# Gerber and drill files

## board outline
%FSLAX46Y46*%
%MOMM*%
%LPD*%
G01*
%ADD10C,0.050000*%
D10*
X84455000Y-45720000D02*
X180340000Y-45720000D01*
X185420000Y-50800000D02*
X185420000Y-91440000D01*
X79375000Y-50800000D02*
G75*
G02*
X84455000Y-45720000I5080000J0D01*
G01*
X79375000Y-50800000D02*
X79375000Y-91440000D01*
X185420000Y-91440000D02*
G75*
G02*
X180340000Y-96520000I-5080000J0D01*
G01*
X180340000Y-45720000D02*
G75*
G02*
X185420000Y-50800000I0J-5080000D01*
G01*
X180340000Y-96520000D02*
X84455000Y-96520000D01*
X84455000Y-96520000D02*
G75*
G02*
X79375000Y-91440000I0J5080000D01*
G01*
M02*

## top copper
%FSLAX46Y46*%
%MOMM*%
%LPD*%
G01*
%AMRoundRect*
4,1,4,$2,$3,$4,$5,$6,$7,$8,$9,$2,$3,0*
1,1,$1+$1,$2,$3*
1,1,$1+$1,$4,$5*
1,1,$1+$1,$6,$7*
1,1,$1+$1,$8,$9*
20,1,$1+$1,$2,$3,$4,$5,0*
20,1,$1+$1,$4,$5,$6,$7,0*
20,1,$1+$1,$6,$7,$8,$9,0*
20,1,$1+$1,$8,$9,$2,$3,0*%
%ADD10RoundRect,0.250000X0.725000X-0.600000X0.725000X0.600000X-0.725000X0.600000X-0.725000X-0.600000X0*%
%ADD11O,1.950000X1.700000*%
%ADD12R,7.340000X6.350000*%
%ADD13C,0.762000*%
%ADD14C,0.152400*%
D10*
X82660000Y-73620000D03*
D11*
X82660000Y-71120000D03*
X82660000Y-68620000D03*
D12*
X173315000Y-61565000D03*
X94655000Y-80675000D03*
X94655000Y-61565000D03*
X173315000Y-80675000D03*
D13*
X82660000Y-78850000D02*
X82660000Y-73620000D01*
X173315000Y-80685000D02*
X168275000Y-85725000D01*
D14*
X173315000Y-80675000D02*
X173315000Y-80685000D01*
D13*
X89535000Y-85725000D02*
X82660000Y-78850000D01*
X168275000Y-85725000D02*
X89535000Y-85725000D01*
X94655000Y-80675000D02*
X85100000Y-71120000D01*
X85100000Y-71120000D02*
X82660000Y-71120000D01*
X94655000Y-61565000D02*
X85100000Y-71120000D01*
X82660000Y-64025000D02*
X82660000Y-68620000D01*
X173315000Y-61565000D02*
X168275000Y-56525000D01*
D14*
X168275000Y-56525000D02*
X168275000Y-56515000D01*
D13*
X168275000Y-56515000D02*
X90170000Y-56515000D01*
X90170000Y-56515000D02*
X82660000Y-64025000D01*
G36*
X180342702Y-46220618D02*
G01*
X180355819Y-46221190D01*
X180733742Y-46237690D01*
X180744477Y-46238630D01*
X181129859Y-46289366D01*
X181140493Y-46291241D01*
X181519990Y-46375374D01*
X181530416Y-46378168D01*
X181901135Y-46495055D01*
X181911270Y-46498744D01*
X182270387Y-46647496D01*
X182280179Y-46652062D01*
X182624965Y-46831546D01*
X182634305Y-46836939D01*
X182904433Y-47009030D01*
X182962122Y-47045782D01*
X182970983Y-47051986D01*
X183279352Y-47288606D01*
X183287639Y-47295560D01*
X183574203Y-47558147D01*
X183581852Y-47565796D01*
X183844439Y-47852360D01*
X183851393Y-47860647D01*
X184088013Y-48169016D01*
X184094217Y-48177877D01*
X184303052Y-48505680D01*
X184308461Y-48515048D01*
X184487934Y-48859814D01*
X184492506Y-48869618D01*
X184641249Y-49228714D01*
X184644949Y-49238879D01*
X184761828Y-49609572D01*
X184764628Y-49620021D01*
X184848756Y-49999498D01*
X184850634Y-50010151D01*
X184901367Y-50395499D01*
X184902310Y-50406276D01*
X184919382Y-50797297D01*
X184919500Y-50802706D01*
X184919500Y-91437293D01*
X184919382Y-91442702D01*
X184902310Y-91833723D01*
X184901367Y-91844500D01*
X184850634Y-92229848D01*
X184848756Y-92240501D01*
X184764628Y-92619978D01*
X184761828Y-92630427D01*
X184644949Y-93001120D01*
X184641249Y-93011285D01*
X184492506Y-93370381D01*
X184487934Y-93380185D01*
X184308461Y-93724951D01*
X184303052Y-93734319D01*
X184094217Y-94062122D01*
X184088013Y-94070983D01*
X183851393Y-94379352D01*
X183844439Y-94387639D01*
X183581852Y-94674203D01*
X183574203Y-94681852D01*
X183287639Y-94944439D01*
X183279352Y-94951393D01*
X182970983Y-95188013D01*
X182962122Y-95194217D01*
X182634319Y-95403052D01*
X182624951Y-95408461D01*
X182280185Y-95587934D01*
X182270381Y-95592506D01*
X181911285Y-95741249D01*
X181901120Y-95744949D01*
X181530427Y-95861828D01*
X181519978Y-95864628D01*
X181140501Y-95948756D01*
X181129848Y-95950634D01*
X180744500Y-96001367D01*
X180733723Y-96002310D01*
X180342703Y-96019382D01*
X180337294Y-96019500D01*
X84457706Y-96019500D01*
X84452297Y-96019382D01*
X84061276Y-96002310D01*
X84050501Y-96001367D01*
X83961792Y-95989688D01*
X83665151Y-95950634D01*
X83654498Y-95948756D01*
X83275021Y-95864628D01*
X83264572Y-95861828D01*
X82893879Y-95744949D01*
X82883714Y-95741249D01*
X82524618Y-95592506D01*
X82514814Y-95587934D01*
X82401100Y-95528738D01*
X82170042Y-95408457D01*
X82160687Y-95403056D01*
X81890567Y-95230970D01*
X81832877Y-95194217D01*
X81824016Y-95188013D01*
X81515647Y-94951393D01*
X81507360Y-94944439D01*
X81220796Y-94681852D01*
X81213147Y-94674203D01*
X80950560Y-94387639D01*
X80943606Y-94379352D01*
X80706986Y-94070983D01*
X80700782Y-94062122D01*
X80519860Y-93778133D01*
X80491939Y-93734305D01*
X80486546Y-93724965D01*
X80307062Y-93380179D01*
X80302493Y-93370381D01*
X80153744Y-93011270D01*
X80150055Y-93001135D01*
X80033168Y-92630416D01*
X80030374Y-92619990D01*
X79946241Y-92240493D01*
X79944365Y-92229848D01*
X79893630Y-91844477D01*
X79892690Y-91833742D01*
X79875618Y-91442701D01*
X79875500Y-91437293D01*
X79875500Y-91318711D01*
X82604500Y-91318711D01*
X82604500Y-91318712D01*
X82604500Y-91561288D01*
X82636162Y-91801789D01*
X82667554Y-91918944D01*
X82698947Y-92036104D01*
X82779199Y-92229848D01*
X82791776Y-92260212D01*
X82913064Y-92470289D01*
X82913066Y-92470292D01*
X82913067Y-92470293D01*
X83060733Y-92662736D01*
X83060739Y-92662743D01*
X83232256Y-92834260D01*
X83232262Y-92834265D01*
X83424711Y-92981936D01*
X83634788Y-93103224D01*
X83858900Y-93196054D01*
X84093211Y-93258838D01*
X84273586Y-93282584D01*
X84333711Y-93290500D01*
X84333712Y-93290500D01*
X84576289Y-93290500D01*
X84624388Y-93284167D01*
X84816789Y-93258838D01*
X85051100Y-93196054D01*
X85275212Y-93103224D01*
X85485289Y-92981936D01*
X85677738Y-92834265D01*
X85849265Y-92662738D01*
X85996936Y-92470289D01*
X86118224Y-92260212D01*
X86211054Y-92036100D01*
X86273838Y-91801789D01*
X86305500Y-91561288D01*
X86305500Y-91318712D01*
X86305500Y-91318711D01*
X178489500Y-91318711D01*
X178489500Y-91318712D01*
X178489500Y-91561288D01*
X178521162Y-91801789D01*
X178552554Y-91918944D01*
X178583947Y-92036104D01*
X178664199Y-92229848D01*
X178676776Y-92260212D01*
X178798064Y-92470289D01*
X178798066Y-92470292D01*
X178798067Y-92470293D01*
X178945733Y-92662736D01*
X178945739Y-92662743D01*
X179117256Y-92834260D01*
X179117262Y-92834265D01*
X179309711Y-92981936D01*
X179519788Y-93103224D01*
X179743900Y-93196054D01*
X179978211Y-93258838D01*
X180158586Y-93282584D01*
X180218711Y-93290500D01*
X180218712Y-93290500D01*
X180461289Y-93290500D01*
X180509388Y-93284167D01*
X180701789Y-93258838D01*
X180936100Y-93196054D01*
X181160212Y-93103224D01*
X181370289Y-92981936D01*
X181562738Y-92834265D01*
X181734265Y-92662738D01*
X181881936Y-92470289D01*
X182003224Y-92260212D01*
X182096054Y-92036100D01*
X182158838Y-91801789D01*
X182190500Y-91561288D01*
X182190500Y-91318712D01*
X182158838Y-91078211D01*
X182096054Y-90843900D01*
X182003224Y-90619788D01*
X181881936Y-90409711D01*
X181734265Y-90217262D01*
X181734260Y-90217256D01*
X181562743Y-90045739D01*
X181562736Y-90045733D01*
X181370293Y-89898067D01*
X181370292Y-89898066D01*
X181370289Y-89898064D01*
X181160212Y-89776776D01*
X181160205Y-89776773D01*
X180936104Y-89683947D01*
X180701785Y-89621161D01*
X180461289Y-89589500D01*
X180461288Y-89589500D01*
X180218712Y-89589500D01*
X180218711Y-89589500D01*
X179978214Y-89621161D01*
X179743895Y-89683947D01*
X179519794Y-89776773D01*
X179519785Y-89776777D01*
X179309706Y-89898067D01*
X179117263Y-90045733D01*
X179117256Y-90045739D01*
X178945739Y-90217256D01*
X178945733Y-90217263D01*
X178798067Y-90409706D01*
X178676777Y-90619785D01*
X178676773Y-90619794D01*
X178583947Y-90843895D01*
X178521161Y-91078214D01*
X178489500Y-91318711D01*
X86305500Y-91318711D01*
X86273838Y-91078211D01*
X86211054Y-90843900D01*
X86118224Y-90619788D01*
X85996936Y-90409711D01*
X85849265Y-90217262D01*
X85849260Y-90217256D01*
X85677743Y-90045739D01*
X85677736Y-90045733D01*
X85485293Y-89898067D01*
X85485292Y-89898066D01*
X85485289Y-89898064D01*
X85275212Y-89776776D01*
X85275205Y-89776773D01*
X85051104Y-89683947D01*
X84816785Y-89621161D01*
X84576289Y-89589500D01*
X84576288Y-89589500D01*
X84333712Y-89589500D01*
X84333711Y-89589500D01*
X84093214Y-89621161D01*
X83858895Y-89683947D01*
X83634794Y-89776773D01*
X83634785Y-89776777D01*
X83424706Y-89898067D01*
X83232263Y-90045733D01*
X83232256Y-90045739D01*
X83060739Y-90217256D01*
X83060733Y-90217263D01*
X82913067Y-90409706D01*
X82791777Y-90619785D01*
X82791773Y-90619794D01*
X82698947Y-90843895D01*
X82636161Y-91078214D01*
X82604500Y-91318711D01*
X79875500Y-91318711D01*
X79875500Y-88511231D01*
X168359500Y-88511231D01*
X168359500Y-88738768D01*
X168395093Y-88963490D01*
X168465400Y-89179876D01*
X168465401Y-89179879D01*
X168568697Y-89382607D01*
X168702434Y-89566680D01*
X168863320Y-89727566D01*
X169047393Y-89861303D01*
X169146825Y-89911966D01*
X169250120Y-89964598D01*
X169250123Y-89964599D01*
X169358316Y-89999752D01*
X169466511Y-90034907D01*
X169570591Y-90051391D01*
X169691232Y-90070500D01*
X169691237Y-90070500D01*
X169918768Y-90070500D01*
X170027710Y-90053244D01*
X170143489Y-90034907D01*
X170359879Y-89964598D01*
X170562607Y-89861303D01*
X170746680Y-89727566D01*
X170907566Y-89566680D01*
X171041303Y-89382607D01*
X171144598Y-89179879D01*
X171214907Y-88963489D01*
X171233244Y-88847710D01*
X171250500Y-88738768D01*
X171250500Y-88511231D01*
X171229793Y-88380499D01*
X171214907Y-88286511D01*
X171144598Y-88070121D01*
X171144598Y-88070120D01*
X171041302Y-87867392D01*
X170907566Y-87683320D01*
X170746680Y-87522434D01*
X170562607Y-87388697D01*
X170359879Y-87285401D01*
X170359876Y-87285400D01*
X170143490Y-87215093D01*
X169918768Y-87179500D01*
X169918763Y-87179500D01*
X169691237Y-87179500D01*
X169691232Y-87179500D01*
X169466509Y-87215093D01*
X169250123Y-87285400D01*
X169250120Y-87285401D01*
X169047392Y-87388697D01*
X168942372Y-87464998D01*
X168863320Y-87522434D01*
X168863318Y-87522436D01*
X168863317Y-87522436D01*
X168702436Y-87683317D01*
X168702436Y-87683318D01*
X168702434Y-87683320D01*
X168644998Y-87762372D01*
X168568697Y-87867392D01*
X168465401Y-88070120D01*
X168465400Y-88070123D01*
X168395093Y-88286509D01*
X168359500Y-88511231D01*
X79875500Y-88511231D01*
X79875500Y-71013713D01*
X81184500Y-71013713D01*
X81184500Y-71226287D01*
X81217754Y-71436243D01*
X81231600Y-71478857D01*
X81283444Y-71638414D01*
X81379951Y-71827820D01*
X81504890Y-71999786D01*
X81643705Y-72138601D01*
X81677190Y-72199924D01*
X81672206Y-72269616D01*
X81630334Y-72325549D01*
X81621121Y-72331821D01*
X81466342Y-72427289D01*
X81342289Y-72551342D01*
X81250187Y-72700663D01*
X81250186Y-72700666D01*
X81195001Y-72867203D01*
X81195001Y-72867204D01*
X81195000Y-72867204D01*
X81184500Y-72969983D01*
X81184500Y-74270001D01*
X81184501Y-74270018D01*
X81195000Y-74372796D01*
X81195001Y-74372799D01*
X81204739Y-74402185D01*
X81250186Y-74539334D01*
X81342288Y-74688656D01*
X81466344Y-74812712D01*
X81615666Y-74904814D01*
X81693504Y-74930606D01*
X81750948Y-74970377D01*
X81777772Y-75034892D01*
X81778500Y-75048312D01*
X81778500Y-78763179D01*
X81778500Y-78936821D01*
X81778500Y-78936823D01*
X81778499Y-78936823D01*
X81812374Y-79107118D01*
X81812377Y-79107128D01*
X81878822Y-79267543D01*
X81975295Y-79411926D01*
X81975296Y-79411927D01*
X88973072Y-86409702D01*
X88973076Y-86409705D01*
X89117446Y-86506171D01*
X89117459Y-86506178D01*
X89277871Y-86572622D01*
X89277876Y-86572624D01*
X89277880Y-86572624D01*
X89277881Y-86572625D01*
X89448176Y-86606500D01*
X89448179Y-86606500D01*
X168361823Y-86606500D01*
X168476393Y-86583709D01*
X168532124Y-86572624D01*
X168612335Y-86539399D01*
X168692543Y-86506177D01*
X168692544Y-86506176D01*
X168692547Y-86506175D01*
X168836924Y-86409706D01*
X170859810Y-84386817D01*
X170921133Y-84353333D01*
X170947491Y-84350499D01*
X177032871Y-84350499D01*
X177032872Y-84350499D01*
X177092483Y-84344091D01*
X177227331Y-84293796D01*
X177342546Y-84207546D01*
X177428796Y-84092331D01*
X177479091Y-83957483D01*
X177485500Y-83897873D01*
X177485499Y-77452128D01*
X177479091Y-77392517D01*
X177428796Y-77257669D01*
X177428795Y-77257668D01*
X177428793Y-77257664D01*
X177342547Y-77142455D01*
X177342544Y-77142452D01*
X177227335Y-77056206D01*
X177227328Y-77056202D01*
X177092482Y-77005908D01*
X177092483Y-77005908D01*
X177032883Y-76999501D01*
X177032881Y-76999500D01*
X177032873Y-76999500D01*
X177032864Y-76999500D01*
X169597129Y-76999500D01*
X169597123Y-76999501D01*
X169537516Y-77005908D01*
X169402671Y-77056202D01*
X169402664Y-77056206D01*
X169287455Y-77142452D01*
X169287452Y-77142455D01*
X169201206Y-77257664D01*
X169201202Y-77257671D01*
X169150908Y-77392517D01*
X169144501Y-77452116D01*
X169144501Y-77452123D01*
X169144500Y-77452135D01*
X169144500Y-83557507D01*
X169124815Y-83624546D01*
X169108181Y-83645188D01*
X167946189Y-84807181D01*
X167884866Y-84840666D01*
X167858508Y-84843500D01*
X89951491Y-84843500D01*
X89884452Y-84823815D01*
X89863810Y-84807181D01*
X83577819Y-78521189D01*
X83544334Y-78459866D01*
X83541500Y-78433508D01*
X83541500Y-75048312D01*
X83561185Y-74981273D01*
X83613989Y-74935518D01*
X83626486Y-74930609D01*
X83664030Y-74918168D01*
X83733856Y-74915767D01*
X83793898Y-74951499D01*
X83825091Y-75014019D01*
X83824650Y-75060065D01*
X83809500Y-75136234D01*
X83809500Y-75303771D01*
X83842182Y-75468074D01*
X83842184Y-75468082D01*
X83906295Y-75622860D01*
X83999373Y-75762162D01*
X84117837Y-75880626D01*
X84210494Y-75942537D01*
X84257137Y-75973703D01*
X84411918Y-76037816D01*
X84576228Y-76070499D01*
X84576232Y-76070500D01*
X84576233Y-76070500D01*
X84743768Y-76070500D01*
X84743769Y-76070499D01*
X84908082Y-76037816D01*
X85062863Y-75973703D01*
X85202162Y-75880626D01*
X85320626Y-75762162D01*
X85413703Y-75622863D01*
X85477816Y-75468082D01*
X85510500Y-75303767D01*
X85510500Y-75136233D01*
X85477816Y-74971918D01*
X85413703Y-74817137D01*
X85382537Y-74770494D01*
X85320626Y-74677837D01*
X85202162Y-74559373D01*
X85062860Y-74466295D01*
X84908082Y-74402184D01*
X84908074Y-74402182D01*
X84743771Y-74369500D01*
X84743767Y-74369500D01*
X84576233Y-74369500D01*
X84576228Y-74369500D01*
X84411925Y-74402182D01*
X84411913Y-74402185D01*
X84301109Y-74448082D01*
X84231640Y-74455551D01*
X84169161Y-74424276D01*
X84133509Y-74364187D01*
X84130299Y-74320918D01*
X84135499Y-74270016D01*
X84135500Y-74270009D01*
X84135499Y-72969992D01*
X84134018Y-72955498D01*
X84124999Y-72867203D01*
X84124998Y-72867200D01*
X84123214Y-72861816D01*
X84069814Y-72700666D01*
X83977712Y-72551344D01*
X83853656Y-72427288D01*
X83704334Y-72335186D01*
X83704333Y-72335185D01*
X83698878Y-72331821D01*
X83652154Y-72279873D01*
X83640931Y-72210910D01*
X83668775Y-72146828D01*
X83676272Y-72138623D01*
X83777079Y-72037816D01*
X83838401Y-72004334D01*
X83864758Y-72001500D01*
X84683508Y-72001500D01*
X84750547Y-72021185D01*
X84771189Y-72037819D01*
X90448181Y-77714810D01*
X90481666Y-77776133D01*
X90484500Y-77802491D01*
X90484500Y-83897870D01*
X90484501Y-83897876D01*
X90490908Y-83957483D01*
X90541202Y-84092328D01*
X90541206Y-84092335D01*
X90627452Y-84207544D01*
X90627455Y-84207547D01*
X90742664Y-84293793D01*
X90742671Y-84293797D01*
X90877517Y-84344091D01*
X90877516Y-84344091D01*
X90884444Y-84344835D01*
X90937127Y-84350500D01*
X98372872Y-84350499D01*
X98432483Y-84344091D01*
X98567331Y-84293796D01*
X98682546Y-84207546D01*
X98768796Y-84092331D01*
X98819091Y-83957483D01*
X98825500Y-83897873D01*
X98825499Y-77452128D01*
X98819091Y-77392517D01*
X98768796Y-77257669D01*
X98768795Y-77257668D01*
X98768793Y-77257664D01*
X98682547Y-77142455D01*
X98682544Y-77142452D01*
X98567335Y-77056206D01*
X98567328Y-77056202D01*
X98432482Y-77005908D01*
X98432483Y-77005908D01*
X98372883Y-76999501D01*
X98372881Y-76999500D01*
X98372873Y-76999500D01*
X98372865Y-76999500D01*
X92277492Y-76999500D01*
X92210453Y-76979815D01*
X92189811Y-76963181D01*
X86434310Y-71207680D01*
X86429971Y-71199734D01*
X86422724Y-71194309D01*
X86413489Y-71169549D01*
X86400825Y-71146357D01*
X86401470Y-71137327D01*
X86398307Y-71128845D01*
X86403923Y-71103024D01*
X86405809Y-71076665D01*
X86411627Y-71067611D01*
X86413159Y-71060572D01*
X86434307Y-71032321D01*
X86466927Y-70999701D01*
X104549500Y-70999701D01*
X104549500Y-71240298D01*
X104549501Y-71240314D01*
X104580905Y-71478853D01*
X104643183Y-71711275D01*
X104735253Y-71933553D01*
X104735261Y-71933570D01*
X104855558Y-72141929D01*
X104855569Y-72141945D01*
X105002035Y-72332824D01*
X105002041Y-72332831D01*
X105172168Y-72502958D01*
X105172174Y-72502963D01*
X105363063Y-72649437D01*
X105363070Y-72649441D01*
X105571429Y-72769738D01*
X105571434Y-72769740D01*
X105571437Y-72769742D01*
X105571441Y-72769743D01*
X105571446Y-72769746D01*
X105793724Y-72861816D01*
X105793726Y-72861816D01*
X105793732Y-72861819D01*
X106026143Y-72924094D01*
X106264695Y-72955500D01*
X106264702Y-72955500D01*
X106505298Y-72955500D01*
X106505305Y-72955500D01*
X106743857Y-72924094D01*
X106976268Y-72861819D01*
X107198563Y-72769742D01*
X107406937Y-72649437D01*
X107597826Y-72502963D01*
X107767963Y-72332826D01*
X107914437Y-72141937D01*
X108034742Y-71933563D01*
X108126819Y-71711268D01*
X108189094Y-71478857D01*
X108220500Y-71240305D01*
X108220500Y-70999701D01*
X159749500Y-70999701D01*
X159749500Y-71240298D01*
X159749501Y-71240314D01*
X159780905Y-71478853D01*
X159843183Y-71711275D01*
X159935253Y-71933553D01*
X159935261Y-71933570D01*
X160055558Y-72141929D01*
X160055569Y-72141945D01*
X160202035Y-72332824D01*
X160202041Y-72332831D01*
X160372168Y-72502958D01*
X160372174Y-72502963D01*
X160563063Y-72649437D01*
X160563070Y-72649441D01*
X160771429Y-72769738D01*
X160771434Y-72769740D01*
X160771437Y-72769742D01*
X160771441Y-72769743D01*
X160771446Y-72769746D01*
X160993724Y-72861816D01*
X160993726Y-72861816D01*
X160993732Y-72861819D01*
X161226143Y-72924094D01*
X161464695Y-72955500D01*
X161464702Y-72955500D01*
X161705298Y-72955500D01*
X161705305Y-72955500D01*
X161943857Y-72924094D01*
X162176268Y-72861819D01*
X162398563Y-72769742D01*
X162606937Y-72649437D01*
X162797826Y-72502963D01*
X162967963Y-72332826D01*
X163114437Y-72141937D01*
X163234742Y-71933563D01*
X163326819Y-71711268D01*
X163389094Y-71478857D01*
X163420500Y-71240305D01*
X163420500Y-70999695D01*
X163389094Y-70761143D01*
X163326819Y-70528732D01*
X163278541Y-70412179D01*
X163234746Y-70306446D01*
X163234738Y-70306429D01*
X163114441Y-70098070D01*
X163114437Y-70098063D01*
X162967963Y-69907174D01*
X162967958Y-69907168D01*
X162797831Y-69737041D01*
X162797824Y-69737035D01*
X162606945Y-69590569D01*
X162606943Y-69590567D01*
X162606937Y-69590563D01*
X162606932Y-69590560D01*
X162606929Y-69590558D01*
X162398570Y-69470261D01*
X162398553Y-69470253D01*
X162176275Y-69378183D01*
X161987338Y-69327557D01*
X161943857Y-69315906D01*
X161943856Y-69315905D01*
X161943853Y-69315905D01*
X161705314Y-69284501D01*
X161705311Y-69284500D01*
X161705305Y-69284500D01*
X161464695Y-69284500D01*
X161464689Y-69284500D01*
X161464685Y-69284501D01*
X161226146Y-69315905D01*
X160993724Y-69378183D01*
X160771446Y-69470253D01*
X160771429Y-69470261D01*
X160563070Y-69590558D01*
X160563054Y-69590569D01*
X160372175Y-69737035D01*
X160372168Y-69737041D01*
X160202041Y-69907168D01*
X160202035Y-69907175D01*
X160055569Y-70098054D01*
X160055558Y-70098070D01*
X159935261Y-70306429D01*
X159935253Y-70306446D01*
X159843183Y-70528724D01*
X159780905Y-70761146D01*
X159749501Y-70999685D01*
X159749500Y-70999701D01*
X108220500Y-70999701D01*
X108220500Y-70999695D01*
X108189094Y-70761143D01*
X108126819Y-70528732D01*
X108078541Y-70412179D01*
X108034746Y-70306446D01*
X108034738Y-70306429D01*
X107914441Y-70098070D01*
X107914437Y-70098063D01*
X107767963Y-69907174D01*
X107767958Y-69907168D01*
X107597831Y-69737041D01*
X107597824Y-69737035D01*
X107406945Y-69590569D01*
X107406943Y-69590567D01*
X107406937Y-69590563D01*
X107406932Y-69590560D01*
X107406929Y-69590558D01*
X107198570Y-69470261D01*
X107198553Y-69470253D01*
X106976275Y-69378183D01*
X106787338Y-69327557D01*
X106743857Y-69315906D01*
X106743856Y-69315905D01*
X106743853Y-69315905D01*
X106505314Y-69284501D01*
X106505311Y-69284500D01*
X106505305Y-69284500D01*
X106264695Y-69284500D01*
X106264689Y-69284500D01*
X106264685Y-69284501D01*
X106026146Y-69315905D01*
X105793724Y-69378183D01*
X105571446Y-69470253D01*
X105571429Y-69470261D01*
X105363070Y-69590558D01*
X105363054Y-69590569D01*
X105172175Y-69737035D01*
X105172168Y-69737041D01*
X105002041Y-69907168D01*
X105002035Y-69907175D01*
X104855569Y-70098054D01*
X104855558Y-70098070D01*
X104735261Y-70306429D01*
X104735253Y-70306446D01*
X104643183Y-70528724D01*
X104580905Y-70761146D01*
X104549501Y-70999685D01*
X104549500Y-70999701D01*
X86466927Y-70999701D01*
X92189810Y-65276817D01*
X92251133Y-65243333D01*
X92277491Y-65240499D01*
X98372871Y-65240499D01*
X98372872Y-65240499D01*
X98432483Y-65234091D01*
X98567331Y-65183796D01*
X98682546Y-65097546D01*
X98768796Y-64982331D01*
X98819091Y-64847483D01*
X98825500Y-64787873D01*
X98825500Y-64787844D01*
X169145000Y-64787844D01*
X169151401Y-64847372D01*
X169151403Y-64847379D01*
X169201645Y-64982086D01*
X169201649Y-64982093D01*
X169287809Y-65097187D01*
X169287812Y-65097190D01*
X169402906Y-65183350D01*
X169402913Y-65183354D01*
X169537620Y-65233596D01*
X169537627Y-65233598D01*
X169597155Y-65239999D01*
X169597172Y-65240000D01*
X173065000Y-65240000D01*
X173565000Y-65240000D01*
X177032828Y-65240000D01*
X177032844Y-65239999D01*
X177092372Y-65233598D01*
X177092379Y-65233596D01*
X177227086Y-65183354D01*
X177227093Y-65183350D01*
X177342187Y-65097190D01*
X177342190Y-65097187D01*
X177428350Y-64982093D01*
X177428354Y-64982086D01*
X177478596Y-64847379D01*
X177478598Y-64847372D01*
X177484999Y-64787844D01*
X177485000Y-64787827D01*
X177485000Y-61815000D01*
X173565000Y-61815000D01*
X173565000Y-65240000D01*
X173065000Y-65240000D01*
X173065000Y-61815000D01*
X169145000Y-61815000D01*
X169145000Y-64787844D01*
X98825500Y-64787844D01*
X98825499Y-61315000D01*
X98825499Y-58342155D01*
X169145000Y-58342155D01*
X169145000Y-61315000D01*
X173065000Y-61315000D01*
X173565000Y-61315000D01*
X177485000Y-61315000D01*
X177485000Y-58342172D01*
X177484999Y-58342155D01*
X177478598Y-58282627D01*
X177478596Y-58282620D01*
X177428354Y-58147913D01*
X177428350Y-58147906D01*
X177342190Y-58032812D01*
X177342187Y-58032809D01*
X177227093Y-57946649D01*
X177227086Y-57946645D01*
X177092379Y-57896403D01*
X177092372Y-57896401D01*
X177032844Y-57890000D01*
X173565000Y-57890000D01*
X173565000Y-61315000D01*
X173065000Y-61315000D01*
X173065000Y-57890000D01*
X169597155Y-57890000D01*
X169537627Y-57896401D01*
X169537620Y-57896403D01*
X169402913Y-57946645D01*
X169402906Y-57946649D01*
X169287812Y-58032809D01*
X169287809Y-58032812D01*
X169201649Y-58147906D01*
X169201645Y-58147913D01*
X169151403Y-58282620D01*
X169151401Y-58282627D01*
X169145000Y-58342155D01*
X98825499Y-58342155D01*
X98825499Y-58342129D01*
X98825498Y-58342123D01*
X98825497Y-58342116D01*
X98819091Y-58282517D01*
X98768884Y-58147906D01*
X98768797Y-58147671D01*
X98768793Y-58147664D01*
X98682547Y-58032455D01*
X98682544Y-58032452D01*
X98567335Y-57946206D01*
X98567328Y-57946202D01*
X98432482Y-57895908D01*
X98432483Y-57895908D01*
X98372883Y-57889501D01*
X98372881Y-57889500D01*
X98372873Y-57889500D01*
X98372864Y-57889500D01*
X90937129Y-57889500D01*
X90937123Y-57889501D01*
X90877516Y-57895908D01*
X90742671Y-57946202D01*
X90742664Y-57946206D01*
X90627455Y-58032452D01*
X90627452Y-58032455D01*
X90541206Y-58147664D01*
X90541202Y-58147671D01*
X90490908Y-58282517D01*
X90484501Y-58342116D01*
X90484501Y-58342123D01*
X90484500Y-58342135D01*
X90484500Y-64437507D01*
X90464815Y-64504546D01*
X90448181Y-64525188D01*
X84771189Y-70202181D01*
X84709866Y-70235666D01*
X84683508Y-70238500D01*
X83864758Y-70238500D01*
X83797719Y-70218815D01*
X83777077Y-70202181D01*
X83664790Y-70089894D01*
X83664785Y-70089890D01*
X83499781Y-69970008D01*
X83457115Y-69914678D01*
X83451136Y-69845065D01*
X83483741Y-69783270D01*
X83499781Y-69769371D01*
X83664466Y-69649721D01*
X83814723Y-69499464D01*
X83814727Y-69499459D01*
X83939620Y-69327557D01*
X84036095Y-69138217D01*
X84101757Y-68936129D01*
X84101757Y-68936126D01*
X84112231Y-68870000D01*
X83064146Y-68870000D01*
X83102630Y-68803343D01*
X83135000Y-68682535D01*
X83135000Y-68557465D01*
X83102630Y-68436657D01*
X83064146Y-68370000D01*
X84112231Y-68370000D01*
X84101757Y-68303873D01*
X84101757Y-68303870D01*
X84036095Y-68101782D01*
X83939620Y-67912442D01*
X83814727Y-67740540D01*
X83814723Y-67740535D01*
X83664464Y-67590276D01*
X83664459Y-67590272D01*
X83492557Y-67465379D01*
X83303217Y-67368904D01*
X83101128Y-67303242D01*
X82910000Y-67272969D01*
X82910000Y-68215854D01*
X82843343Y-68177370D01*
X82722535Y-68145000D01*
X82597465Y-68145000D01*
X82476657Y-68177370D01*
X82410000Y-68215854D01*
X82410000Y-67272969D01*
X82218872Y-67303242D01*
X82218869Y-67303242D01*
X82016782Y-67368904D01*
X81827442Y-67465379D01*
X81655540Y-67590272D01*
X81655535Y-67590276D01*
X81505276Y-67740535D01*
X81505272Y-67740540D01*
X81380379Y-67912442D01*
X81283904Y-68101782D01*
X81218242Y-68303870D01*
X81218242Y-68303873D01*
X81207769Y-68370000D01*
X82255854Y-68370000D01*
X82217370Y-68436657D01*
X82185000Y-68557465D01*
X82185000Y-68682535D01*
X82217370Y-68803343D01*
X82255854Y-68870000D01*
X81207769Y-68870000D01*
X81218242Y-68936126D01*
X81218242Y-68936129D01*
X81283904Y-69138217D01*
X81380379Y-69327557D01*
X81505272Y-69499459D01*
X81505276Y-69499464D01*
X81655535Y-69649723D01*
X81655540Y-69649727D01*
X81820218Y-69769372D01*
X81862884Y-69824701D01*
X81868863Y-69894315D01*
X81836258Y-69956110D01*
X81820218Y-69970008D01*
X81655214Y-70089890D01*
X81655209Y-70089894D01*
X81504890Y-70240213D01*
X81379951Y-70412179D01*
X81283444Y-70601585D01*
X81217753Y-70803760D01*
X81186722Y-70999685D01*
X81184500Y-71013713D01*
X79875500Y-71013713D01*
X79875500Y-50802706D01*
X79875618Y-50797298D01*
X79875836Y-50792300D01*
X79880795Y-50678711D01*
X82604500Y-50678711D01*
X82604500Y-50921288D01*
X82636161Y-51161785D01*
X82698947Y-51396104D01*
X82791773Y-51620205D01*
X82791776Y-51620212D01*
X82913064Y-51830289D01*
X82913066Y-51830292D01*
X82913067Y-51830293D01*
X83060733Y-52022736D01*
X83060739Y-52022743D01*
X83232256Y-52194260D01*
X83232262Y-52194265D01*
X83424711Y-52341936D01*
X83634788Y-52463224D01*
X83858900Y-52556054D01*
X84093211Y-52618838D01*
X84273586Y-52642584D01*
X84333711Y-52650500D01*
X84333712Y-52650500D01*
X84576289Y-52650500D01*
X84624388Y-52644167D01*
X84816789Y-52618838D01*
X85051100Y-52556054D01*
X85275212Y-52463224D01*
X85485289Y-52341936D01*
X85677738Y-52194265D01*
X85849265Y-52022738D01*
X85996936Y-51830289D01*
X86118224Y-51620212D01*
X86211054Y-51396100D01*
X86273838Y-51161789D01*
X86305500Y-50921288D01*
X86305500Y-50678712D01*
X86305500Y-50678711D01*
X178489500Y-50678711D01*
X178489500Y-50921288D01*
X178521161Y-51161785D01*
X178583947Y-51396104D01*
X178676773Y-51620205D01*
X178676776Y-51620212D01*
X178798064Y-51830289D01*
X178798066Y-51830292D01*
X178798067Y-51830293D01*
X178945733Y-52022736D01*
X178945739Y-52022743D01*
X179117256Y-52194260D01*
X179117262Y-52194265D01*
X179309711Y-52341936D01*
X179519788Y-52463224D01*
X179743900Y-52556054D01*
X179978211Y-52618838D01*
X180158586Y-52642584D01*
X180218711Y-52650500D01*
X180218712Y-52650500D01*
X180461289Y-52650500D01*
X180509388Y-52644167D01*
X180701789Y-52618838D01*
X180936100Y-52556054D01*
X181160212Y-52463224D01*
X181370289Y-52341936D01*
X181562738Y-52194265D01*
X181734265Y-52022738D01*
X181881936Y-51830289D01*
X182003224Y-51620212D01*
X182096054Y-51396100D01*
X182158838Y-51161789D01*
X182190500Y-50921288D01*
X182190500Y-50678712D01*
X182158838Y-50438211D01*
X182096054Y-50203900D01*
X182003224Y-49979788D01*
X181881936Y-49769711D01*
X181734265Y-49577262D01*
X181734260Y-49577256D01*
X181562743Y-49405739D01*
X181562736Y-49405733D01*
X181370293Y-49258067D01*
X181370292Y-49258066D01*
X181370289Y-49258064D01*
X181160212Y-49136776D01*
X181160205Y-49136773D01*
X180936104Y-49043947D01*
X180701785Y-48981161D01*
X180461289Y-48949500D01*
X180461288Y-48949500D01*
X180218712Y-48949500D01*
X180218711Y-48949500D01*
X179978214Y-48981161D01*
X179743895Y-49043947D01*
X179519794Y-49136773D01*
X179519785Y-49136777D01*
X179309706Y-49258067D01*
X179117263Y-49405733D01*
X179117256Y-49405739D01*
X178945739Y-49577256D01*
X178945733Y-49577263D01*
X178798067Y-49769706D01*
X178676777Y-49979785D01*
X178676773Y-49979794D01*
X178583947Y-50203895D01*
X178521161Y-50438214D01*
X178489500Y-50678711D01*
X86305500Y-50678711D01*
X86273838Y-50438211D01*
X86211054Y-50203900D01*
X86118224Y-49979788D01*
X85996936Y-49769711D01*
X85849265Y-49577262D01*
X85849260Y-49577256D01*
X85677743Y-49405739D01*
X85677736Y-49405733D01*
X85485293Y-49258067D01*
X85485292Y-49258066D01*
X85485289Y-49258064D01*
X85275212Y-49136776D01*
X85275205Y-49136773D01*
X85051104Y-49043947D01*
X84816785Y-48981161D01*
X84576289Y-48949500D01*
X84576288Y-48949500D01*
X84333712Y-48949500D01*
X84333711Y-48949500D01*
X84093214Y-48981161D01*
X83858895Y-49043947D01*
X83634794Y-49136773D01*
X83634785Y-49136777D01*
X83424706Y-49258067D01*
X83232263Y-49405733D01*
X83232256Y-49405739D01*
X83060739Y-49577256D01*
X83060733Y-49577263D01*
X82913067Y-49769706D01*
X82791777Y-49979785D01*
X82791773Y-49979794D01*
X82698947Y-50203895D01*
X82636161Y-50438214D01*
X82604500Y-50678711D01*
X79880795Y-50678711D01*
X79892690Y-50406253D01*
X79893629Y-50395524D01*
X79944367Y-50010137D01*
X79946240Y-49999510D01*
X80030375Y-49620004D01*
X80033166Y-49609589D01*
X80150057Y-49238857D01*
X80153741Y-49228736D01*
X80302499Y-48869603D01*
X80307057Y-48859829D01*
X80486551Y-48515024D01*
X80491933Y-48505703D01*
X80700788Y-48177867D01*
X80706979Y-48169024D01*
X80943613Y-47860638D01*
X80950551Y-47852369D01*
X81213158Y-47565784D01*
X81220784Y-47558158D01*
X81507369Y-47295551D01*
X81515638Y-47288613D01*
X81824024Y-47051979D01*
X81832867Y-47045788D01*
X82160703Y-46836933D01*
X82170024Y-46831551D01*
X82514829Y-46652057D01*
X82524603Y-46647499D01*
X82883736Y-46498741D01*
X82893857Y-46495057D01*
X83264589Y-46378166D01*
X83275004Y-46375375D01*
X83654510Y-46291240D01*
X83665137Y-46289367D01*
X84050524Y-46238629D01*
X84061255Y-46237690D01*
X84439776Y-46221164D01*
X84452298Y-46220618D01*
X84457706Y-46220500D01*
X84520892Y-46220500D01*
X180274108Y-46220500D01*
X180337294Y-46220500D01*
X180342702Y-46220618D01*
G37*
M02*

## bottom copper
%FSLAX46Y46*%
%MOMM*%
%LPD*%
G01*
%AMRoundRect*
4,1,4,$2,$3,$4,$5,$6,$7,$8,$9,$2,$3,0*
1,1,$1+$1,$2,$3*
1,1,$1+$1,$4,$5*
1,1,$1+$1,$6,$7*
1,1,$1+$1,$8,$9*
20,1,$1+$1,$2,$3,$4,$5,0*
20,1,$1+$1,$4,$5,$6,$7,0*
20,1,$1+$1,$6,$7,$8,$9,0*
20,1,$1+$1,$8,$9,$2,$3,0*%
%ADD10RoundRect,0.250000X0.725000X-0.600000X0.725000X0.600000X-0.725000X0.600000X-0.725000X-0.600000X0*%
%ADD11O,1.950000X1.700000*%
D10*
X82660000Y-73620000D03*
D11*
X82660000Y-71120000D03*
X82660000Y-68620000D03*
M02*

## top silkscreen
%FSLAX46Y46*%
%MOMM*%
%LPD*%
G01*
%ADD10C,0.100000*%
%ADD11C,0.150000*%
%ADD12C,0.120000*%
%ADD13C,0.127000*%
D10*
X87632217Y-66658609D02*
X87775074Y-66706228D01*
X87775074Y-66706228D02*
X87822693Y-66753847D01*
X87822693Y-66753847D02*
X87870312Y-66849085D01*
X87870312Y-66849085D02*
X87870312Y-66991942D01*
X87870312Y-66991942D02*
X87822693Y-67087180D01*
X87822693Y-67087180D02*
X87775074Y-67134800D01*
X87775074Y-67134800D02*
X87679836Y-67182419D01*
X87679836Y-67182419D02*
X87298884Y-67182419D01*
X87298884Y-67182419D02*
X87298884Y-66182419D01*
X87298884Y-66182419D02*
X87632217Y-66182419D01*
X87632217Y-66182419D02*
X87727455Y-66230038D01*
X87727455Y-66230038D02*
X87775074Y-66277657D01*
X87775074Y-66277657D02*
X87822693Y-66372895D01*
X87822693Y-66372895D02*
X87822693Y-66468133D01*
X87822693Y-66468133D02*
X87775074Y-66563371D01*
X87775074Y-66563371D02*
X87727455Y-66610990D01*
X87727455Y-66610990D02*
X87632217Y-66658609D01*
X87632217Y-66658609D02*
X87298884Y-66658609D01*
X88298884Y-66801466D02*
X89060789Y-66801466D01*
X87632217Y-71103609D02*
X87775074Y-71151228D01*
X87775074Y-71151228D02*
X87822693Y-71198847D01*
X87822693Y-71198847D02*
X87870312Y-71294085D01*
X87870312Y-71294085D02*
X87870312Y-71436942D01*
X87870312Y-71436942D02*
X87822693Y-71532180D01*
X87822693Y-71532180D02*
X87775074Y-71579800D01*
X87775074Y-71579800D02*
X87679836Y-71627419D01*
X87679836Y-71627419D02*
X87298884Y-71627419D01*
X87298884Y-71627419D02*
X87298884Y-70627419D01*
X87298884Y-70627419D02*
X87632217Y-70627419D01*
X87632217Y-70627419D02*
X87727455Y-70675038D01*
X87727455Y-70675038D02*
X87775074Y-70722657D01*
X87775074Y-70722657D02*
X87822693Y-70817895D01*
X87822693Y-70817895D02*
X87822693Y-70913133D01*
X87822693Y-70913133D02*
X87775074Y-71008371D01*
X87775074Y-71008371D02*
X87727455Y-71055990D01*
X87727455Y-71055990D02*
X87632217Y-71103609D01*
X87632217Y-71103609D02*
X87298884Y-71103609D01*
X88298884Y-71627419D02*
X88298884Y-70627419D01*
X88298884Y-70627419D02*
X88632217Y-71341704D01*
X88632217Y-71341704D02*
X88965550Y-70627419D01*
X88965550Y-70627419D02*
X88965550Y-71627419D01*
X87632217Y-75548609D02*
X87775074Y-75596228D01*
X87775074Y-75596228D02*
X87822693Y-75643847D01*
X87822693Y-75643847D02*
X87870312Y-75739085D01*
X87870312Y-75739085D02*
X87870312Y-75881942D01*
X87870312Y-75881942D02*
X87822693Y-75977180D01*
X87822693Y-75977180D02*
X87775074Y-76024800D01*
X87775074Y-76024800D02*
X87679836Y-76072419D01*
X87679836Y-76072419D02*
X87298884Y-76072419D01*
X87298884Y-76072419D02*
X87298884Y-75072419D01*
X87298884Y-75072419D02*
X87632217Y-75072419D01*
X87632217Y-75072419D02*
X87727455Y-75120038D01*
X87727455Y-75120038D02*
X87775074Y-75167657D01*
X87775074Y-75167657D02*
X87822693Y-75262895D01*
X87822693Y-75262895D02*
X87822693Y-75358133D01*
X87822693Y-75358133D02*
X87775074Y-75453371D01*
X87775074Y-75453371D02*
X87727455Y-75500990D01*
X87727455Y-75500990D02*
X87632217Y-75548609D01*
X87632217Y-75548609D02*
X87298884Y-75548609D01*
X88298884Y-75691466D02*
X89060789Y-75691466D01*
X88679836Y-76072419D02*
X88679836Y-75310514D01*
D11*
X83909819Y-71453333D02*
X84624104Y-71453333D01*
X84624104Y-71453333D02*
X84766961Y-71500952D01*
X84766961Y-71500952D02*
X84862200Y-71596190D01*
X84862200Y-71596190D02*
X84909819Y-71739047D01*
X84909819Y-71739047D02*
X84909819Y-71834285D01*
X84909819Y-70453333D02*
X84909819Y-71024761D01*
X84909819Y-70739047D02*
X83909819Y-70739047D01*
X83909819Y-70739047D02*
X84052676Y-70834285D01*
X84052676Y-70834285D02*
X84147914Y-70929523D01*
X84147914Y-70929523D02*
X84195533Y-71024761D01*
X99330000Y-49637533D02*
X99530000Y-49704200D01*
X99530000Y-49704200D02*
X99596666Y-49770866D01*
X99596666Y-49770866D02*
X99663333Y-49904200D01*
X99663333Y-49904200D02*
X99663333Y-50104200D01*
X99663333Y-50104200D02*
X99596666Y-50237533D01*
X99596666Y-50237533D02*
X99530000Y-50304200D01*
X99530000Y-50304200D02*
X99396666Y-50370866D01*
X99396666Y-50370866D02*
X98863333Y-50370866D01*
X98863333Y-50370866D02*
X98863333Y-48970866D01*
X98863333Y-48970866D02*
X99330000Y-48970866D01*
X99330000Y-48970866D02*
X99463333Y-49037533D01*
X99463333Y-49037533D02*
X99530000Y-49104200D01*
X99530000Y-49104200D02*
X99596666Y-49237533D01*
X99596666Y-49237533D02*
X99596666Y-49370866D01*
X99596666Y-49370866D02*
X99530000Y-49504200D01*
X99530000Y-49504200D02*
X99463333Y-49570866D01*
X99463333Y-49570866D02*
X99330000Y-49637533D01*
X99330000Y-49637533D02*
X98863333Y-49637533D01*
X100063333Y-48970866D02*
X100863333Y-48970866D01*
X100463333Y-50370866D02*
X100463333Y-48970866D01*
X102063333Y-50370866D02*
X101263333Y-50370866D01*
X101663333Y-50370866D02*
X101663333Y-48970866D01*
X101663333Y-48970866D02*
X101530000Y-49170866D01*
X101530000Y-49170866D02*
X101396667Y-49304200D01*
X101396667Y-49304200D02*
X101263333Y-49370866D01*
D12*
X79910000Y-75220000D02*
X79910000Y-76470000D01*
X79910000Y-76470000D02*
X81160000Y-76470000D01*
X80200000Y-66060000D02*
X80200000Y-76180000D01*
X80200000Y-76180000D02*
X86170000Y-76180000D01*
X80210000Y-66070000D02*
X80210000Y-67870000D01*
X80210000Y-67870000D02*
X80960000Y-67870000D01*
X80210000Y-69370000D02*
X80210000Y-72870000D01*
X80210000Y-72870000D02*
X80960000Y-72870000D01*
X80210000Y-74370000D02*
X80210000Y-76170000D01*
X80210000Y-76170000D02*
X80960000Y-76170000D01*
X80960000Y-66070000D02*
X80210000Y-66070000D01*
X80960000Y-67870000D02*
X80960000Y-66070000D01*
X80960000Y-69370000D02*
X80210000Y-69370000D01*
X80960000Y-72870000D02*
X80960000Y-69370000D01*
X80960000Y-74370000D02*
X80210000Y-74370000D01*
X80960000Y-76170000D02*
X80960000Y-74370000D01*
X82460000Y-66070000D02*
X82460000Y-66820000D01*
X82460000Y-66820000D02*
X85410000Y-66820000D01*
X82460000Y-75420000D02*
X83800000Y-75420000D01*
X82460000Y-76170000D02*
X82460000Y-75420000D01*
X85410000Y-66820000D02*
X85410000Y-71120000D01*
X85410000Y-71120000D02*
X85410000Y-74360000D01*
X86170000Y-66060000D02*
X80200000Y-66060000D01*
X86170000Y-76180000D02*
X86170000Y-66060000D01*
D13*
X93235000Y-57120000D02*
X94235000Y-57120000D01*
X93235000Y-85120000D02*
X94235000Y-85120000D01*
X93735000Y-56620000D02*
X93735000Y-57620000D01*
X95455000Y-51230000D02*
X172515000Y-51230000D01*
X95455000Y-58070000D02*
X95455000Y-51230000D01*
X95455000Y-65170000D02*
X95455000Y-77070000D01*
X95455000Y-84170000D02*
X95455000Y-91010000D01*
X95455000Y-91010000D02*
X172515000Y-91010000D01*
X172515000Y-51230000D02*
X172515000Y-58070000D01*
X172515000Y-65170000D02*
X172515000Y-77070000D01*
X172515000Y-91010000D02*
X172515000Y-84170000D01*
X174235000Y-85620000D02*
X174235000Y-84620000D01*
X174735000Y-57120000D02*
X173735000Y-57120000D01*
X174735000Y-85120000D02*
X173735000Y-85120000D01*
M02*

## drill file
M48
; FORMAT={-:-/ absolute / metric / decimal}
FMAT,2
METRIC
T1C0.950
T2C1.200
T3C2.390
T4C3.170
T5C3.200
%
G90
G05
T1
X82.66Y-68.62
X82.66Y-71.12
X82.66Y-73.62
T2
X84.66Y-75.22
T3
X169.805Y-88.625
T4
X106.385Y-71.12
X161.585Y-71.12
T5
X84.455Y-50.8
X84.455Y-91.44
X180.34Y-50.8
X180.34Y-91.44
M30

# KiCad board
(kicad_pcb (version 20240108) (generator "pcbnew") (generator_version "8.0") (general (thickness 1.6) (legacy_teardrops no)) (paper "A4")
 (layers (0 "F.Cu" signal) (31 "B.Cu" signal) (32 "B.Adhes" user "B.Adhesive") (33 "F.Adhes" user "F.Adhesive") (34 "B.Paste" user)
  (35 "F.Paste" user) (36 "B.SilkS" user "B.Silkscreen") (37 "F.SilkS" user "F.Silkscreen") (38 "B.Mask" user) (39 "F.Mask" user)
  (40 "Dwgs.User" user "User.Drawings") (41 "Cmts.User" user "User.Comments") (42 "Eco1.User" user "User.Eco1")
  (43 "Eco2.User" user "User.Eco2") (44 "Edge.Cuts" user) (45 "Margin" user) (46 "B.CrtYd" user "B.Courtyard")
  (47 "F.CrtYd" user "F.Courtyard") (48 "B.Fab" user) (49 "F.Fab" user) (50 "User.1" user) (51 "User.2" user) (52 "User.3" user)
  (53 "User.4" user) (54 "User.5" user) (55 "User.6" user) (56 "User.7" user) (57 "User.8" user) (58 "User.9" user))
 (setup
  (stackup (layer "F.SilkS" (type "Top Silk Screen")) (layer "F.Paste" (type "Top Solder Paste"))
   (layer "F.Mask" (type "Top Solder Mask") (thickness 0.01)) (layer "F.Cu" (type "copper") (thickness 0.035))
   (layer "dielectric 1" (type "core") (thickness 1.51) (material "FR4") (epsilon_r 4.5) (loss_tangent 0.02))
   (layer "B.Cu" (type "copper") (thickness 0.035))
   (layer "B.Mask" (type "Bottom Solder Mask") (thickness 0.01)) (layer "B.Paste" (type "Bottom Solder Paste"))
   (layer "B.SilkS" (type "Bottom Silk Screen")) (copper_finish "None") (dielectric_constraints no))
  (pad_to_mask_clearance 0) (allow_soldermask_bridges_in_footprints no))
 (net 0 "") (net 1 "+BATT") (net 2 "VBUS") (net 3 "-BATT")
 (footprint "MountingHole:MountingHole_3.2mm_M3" (layer "F.Cu") (at 84.455 50.8)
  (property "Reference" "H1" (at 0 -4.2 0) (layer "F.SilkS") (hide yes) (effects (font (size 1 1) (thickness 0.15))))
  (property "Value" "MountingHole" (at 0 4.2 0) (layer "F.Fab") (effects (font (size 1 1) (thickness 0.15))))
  (pad "" np_thru_hole circle (at 0 0) (size 3.2 3.2) (drill 3.2) (layers "*.Cu" "*.Mask")))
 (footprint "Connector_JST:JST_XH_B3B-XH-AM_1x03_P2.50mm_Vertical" (layer "F.Cu") (at 82.66 73.62 90)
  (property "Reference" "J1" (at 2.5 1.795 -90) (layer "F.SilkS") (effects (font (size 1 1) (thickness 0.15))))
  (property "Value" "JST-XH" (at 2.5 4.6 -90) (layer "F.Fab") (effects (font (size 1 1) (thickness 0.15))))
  (fp_line (start -1.6 -2.75) (end -2.85 -2.75) (stroke (width 0.12) (type solid)) (layer "F.SilkS"))
  (fp_line (start -2.85 -2.75) (end -2.85 -1.5) (stroke (width 0.12) (type solid)) (layer "F.SilkS"))
  (fp_line (start 7.56 -2.46) (end -2.56 -2.46) (stroke (width 0.12) (type solid)) (layer "F.SilkS"))
  (fp_line (start -2.56 -2.46) (end -2.56 3.51) (stroke (width 0.12) (type solid)) (layer "F.SilkS"))
  (fp_line (start 7.55 -2.45) (end 5.75 -2.45) (stroke (width 0.12) (type solid)) (layer "F.SilkS"))
  (fp_line (start 5.75 -2.45) (end 5.75 -1.7) (stroke (width 0.12) (type solid)) (layer "F.SilkS"))
  (fp_line (start 4.25 -2.45) (end 0.75 -2.45) (stroke (width 0.12) (type solid)) (layer "F.SilkS"))
  (fp_line (start 0.75 -2.45) (end 0.75 -1.7) (stroke (width 0.12) (type solid)) (layer "F.SilkS"))
  (fp_line (start -0.75 -2.45) (end -2.55 -2.45) (stroke (width 0.12) (type solid)) (layer "F.SilkS"))
  (fp_line (start -2.55 -2.45) (end -2.55 -1.7) (stroke (width 0.12) (type solid)) (layer "F.SilkS"))
  (fp_line (start 7.55 -1.7) (end 7.55 -2.45) (stroke (width 0.12) (type solid)) (layer "F.SilkS"))
  (fp_line (start 5.75 -1.7) (end 7.55 -1.7) (stroke (width 0.12) (type solid)) (layer "F.SilkS"))
  (fp_line (start 4.25 -1.7) (end 4.25 -2.45) (stroke (width 0.12) (type solid)) (layer "F.SilkS"))
  (fp_line (start 0.75 -1.7) (end 4.25 -1.7) (stroke (width 0.12) (type solid)) (layer "F.SilkS"))
  (fp_line (start -0.75 -1.7) (end -0.75 -2.45) (stroke (width 0.12) (type solid)) (layer "F.SilkS"))
  (fp_line (start -2.55 -1.7) (end -0.75 -1.7) (stroke (width 0.12) (type solid)) (layer "F.SilkS"))
  (fp_line (start 7.55 -0.2) (end 6.8 -0.2) (stroke (width 0.12) (type solid)) (layer "F.SilkS"))
  (fp_line (start 6.8 -0.2) (end 6.8 2.75) (stroke (width 0.12) (type solid)) (layer "F.SilkS"))
  (fp_line (start -1.8 -0.2) (end -1.8 1.14) (stroke (width 0.12) (type solid)) (layer "F.SilkS"))
  (fp_line (start -2.55 -0.2) (end -1.8 -0.2) (stroke (width 0.12) (type solid)) (layer "F.SilkS"))
  (fp_line (start 6.8 2.75) (end 2.5 2.75) (stroke (width 0.12) (type solid)) (layer "F.SilkS"))
  (fp_line (start 2.5 2.75) (end -0.74 2.75) (stroke (width 0.12) (type solid)) (layer "F.SilkS"))
  (fp_line (start 7.56 3.51) (end 7.56 -2.46) (stroke (width 0.12) (type solid)) (layer "F.SilkS"))
  (fp_line (start -2.56 3.51) (end 7.56 3.51) (stroke (width 0.12) (type solid)) (layer "F.SilkS"))
  (pad "" np_thru_hole circle (at -1.6 2 90) (size 1.2 1.2) (drill 1.2) (layers "*.Cu" "*.Mask"))
  (pad "1" thru_hole roundrect (at 0 0 90) (size 1.7 1.95) (drill 0.95) (layers "*.Cu" "*.Mask") (remove_unused_layers no)
   (roundrect_rratio 0.1470588235) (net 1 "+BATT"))
  (pad "2" thru_hole oval (at 2.5 0 90) (size 1.7 1.95) (drill 0.95) (layers "*.Cu" "*.Mask") (remove_unused_layers no) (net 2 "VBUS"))
  (pad "3" thru_hole oval (at 5 0 90) (size 1.7 1.95) (drill 0.95) (layers "*.Cu" "*.Mask") (remove_unused_layers no) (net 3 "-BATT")))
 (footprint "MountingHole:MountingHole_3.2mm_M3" (layer "F.Cu") (at 180.34 91.44)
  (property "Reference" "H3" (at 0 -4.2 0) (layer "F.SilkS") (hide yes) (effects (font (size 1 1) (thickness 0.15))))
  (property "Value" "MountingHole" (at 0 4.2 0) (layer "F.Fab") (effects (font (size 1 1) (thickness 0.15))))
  (pad "" np_thru_hole circle (at 0 0) (size 3.2 3.2) (drill 3.2) (layers "*.Cu" "*.Mask")))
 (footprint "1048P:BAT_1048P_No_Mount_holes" (layer "F.Cu") (at 133.985 71.12)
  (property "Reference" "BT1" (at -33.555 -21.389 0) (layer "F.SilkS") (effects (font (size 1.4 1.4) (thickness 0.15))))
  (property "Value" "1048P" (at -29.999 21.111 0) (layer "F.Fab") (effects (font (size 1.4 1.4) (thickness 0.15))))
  (fp_line (start -40.75 -14) (end -39.75 -14) (stroke (width 0.127) (type solid)) (layer "F.SilkS"))
  (fp_line (start -40.75 14) (end -39.75 14) (stroke (width 0.127) (type solid)) (layer "F.SilkS"))
  (fp_line (start -40.25 -14.5) (end -40.25 -13.5) (stroke (width 0.127) (type solid)) (layer "F.SilkS"))
  (fp_line (start -38.53 -19.89) (end 38.53 -19.89) (stroke (width 0.127) (type solid)) (layer "F.SilkS"))
  (fp_line (start -38.53 -13.05) (end -38.53 -19.89) (stroke (width 0.127) (type solid)) (layer "F.SilkS"))
  (fp_line (start -38.53 -5.95) (end -38.53 5.95) (stroke (width 0.127) (type solid)) (layer "F.SilkS"))
  (fp_line (start -38.53 13.05) (end -38.53 19.89) (stroke (width 0.127) (type solid)) (layer "F.SilkS"))
  (fp_line (start -38.53 19.89) (end 38.53 19.89) (stroke (width 0.127) (type solid)) (layer "F.SilkS"))
  (fp_line (start 38.53 -19.89) (end 38.53 -13.05) (stroke (width 0.127) (type solid)) (layer "F.SilkS"))
  (fp_line (start 38.53 -5.95) (end 38.53 5.95) (stroke (width 0.127) (type solid)) (layer "F.SilkS"))
  (fp_line (start 38.53 19.89) (end 38.53 13.05) (stroke (width 0.127) (type solid)) (layer "F.SilkS"))
  (fp_line (start 40.25 14.5) (end 40.25 13.5) (stroke (width 0.127) (type solid)) (layer "F.SilkS"))
  (fp_line (start 40.75 -14) (end 39.75 -14) (stroke (width 0.127) (type solid)) (layer "F.SilkS"))
  (fp_line (start 40.75 14) (end 39.75 14) (stroke (width 0.127) (type solid)) (layer "F.SilkS"))
  (pad "" np_thru_hole circle (at -27.6 0) (size 3.17 3.17) (drill 3.17) (layers "*.Cu" "*.Mask"))
  (pad "" np_thru_hole circle (at 27.6 0) (size 3.17 3.17) (drill 3.17) (layers "*.Cu" "*.Mask"))
  (pad "" np_thru_hole circle (at 35.82 17.505) (size 2.39 2.39) (drill 2.39) (layers "*.Cu" "*.Mask"))
  (pad "N1" smd rect (at 39.33 -9.555) (size 7.34 6.35) (layers "F.Cu" "F.Paste" "F.Mask") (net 3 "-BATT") (solder_mask_margin 0.102))
  (pad "N2" smd rect (at -39.33 9.555) (size 7.34 6.35) (layers "F.Cu" "F.Paste" "F.Mask") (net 2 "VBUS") (solder_mask_margin 0.102))
  (pad "P1" smd rect (at -39.33 -9.555) (size 7.34 6.35) (layers "F.Cu" "F.Paste" "F.Mask") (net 2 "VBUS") (solder_mask_margin 0.102))
  (pad "P2" smd rect (at 39.33 9.555) (size 7.34 6.35) (layers "F.Cu" "F.Paste" "F.Mask") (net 1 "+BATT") (solder_mask_margin 0.102)))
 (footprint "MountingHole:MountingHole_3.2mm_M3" (layer "F.Cu") (at 84.455 91.44)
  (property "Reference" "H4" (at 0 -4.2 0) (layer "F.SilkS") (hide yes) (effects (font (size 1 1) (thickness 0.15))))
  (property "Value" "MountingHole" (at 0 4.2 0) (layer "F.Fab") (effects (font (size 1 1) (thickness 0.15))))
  (pad "" np_thru_hole circle (at 0 0) (size 3.2 3.2) (drill 3.2) (layers "*.Cu" "*.Mask")))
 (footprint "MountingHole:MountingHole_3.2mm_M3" (layer "F.Cu") (at 180.34 50.8)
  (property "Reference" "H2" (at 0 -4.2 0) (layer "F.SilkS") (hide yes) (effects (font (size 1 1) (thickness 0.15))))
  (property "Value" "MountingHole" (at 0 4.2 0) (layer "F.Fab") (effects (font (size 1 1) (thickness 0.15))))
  (pad "" np_thru_hole circle (at 0 0) (size 3.2 3.2) (drill 3.2) (layers "*.Cu" "*.Mask")))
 (gr_line (start 84.455 45.72) (end 180.34 45.72) (stroke (width 0.05) (type default)) (layer "Edge.Cuts"))
 (gr_line (start 185.42 50.8) (end 185.42 91.44) (stroke (width 0.05) (type default)) (layer "Edge.Cuts"))
 (gr_arc (start 79.375 50.8) (mid 80.862898 47.207898) (end 84.455 45.72) (stroke (width 0.05) (type default)) (layer "Edge.Cuts"))
 (gr_line (start 79.375 50.8) (end 79.375 91.44) (stroke (width 0.05) (type default)) (layer "Edge.Cuts"))
 (gr_arc (start 185.42 91.44) (mid 183.932102 95.032102) (end 180.34 96.52) (stroke (width 0.05) (type default)) (layer "Edge.Cuts"))
 (gr_arc (start 180.34 45.72) (mid 183.932102 47.207898) (end 185.42 50.8) (stroke (width 0.05) (type default)) (layer "Edge.Cuts"))
 (gr_line (start 180.34 96.52) (end 84.455 96.52) (stroke (width 0.05) (type default)) (layer "Edge.Cuts"))
 (gr_arc (start 84.455 96.52) (mid 80.862898 95.032102) (end 79.375 91.44) (stroke (width 0.05) (type default)) (layer "Edge.Cuts"))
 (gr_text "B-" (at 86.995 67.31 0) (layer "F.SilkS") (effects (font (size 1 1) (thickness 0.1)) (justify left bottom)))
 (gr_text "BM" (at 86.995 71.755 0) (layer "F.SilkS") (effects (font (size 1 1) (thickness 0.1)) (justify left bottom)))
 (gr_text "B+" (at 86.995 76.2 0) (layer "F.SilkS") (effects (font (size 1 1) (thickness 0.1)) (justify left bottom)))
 (segment (start 82.66 78.85) (end 82.66 73.62) (width 0.762) (layer "F.Cu") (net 1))
 (segment (start 173.315 80.685) (end 168.275 85.725) (width 0.762) (layer "F.Cu") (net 1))
 (segment (start 173.315 80.675) (end 173.315 80.685) (width 0.1524) (layer "F.Cu") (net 1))
 (segment (start 89.535 85.725) (end 82.66 78.85) (width 0.762) (layer "F.Cu") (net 1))
 (segment (start 168.275 85.725) (end 89.535 85.725) (width 0.762) (layer "F.Cu") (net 1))
 (segment (start 94.655 80.675) (end 85.1 71.12) (width 0.762) (layer "F.Cu") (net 2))
 (segment (start 85.1 71.12) (end 82.66 71.12) (width 0.762) (layer "F.Cu") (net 2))
 (segment (start 94.655 61.565) (end 85.1 71.12) (width 0.762) (layer "F.Cu") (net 2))
 (segment (start 82.66 64.025) (end 82.66 68.62) (width 0.762) (layer "F.Cu") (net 3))
 (segment (start 173.315 61.565) (end 168.275 56.525) (width 0.762) (layer "F.Cu") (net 3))
 (segment (start 168.275 56.525) (end 168.275 56.515) (width 0.1524) (layer "F.Cu") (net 3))
 (segment (start 168.275 56.515) (end 90.17 56.515) (width 0.762) (layer "F.Cu") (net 3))
 (segment (start 90.17 56.515) (end 82.66 64.025) (width 0.762) (layer "F.Cu") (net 3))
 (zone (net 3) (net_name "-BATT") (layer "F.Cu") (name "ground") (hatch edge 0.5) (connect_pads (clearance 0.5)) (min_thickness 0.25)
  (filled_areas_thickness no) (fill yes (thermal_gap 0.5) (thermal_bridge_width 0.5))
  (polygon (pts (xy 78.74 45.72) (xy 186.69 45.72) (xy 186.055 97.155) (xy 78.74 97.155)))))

